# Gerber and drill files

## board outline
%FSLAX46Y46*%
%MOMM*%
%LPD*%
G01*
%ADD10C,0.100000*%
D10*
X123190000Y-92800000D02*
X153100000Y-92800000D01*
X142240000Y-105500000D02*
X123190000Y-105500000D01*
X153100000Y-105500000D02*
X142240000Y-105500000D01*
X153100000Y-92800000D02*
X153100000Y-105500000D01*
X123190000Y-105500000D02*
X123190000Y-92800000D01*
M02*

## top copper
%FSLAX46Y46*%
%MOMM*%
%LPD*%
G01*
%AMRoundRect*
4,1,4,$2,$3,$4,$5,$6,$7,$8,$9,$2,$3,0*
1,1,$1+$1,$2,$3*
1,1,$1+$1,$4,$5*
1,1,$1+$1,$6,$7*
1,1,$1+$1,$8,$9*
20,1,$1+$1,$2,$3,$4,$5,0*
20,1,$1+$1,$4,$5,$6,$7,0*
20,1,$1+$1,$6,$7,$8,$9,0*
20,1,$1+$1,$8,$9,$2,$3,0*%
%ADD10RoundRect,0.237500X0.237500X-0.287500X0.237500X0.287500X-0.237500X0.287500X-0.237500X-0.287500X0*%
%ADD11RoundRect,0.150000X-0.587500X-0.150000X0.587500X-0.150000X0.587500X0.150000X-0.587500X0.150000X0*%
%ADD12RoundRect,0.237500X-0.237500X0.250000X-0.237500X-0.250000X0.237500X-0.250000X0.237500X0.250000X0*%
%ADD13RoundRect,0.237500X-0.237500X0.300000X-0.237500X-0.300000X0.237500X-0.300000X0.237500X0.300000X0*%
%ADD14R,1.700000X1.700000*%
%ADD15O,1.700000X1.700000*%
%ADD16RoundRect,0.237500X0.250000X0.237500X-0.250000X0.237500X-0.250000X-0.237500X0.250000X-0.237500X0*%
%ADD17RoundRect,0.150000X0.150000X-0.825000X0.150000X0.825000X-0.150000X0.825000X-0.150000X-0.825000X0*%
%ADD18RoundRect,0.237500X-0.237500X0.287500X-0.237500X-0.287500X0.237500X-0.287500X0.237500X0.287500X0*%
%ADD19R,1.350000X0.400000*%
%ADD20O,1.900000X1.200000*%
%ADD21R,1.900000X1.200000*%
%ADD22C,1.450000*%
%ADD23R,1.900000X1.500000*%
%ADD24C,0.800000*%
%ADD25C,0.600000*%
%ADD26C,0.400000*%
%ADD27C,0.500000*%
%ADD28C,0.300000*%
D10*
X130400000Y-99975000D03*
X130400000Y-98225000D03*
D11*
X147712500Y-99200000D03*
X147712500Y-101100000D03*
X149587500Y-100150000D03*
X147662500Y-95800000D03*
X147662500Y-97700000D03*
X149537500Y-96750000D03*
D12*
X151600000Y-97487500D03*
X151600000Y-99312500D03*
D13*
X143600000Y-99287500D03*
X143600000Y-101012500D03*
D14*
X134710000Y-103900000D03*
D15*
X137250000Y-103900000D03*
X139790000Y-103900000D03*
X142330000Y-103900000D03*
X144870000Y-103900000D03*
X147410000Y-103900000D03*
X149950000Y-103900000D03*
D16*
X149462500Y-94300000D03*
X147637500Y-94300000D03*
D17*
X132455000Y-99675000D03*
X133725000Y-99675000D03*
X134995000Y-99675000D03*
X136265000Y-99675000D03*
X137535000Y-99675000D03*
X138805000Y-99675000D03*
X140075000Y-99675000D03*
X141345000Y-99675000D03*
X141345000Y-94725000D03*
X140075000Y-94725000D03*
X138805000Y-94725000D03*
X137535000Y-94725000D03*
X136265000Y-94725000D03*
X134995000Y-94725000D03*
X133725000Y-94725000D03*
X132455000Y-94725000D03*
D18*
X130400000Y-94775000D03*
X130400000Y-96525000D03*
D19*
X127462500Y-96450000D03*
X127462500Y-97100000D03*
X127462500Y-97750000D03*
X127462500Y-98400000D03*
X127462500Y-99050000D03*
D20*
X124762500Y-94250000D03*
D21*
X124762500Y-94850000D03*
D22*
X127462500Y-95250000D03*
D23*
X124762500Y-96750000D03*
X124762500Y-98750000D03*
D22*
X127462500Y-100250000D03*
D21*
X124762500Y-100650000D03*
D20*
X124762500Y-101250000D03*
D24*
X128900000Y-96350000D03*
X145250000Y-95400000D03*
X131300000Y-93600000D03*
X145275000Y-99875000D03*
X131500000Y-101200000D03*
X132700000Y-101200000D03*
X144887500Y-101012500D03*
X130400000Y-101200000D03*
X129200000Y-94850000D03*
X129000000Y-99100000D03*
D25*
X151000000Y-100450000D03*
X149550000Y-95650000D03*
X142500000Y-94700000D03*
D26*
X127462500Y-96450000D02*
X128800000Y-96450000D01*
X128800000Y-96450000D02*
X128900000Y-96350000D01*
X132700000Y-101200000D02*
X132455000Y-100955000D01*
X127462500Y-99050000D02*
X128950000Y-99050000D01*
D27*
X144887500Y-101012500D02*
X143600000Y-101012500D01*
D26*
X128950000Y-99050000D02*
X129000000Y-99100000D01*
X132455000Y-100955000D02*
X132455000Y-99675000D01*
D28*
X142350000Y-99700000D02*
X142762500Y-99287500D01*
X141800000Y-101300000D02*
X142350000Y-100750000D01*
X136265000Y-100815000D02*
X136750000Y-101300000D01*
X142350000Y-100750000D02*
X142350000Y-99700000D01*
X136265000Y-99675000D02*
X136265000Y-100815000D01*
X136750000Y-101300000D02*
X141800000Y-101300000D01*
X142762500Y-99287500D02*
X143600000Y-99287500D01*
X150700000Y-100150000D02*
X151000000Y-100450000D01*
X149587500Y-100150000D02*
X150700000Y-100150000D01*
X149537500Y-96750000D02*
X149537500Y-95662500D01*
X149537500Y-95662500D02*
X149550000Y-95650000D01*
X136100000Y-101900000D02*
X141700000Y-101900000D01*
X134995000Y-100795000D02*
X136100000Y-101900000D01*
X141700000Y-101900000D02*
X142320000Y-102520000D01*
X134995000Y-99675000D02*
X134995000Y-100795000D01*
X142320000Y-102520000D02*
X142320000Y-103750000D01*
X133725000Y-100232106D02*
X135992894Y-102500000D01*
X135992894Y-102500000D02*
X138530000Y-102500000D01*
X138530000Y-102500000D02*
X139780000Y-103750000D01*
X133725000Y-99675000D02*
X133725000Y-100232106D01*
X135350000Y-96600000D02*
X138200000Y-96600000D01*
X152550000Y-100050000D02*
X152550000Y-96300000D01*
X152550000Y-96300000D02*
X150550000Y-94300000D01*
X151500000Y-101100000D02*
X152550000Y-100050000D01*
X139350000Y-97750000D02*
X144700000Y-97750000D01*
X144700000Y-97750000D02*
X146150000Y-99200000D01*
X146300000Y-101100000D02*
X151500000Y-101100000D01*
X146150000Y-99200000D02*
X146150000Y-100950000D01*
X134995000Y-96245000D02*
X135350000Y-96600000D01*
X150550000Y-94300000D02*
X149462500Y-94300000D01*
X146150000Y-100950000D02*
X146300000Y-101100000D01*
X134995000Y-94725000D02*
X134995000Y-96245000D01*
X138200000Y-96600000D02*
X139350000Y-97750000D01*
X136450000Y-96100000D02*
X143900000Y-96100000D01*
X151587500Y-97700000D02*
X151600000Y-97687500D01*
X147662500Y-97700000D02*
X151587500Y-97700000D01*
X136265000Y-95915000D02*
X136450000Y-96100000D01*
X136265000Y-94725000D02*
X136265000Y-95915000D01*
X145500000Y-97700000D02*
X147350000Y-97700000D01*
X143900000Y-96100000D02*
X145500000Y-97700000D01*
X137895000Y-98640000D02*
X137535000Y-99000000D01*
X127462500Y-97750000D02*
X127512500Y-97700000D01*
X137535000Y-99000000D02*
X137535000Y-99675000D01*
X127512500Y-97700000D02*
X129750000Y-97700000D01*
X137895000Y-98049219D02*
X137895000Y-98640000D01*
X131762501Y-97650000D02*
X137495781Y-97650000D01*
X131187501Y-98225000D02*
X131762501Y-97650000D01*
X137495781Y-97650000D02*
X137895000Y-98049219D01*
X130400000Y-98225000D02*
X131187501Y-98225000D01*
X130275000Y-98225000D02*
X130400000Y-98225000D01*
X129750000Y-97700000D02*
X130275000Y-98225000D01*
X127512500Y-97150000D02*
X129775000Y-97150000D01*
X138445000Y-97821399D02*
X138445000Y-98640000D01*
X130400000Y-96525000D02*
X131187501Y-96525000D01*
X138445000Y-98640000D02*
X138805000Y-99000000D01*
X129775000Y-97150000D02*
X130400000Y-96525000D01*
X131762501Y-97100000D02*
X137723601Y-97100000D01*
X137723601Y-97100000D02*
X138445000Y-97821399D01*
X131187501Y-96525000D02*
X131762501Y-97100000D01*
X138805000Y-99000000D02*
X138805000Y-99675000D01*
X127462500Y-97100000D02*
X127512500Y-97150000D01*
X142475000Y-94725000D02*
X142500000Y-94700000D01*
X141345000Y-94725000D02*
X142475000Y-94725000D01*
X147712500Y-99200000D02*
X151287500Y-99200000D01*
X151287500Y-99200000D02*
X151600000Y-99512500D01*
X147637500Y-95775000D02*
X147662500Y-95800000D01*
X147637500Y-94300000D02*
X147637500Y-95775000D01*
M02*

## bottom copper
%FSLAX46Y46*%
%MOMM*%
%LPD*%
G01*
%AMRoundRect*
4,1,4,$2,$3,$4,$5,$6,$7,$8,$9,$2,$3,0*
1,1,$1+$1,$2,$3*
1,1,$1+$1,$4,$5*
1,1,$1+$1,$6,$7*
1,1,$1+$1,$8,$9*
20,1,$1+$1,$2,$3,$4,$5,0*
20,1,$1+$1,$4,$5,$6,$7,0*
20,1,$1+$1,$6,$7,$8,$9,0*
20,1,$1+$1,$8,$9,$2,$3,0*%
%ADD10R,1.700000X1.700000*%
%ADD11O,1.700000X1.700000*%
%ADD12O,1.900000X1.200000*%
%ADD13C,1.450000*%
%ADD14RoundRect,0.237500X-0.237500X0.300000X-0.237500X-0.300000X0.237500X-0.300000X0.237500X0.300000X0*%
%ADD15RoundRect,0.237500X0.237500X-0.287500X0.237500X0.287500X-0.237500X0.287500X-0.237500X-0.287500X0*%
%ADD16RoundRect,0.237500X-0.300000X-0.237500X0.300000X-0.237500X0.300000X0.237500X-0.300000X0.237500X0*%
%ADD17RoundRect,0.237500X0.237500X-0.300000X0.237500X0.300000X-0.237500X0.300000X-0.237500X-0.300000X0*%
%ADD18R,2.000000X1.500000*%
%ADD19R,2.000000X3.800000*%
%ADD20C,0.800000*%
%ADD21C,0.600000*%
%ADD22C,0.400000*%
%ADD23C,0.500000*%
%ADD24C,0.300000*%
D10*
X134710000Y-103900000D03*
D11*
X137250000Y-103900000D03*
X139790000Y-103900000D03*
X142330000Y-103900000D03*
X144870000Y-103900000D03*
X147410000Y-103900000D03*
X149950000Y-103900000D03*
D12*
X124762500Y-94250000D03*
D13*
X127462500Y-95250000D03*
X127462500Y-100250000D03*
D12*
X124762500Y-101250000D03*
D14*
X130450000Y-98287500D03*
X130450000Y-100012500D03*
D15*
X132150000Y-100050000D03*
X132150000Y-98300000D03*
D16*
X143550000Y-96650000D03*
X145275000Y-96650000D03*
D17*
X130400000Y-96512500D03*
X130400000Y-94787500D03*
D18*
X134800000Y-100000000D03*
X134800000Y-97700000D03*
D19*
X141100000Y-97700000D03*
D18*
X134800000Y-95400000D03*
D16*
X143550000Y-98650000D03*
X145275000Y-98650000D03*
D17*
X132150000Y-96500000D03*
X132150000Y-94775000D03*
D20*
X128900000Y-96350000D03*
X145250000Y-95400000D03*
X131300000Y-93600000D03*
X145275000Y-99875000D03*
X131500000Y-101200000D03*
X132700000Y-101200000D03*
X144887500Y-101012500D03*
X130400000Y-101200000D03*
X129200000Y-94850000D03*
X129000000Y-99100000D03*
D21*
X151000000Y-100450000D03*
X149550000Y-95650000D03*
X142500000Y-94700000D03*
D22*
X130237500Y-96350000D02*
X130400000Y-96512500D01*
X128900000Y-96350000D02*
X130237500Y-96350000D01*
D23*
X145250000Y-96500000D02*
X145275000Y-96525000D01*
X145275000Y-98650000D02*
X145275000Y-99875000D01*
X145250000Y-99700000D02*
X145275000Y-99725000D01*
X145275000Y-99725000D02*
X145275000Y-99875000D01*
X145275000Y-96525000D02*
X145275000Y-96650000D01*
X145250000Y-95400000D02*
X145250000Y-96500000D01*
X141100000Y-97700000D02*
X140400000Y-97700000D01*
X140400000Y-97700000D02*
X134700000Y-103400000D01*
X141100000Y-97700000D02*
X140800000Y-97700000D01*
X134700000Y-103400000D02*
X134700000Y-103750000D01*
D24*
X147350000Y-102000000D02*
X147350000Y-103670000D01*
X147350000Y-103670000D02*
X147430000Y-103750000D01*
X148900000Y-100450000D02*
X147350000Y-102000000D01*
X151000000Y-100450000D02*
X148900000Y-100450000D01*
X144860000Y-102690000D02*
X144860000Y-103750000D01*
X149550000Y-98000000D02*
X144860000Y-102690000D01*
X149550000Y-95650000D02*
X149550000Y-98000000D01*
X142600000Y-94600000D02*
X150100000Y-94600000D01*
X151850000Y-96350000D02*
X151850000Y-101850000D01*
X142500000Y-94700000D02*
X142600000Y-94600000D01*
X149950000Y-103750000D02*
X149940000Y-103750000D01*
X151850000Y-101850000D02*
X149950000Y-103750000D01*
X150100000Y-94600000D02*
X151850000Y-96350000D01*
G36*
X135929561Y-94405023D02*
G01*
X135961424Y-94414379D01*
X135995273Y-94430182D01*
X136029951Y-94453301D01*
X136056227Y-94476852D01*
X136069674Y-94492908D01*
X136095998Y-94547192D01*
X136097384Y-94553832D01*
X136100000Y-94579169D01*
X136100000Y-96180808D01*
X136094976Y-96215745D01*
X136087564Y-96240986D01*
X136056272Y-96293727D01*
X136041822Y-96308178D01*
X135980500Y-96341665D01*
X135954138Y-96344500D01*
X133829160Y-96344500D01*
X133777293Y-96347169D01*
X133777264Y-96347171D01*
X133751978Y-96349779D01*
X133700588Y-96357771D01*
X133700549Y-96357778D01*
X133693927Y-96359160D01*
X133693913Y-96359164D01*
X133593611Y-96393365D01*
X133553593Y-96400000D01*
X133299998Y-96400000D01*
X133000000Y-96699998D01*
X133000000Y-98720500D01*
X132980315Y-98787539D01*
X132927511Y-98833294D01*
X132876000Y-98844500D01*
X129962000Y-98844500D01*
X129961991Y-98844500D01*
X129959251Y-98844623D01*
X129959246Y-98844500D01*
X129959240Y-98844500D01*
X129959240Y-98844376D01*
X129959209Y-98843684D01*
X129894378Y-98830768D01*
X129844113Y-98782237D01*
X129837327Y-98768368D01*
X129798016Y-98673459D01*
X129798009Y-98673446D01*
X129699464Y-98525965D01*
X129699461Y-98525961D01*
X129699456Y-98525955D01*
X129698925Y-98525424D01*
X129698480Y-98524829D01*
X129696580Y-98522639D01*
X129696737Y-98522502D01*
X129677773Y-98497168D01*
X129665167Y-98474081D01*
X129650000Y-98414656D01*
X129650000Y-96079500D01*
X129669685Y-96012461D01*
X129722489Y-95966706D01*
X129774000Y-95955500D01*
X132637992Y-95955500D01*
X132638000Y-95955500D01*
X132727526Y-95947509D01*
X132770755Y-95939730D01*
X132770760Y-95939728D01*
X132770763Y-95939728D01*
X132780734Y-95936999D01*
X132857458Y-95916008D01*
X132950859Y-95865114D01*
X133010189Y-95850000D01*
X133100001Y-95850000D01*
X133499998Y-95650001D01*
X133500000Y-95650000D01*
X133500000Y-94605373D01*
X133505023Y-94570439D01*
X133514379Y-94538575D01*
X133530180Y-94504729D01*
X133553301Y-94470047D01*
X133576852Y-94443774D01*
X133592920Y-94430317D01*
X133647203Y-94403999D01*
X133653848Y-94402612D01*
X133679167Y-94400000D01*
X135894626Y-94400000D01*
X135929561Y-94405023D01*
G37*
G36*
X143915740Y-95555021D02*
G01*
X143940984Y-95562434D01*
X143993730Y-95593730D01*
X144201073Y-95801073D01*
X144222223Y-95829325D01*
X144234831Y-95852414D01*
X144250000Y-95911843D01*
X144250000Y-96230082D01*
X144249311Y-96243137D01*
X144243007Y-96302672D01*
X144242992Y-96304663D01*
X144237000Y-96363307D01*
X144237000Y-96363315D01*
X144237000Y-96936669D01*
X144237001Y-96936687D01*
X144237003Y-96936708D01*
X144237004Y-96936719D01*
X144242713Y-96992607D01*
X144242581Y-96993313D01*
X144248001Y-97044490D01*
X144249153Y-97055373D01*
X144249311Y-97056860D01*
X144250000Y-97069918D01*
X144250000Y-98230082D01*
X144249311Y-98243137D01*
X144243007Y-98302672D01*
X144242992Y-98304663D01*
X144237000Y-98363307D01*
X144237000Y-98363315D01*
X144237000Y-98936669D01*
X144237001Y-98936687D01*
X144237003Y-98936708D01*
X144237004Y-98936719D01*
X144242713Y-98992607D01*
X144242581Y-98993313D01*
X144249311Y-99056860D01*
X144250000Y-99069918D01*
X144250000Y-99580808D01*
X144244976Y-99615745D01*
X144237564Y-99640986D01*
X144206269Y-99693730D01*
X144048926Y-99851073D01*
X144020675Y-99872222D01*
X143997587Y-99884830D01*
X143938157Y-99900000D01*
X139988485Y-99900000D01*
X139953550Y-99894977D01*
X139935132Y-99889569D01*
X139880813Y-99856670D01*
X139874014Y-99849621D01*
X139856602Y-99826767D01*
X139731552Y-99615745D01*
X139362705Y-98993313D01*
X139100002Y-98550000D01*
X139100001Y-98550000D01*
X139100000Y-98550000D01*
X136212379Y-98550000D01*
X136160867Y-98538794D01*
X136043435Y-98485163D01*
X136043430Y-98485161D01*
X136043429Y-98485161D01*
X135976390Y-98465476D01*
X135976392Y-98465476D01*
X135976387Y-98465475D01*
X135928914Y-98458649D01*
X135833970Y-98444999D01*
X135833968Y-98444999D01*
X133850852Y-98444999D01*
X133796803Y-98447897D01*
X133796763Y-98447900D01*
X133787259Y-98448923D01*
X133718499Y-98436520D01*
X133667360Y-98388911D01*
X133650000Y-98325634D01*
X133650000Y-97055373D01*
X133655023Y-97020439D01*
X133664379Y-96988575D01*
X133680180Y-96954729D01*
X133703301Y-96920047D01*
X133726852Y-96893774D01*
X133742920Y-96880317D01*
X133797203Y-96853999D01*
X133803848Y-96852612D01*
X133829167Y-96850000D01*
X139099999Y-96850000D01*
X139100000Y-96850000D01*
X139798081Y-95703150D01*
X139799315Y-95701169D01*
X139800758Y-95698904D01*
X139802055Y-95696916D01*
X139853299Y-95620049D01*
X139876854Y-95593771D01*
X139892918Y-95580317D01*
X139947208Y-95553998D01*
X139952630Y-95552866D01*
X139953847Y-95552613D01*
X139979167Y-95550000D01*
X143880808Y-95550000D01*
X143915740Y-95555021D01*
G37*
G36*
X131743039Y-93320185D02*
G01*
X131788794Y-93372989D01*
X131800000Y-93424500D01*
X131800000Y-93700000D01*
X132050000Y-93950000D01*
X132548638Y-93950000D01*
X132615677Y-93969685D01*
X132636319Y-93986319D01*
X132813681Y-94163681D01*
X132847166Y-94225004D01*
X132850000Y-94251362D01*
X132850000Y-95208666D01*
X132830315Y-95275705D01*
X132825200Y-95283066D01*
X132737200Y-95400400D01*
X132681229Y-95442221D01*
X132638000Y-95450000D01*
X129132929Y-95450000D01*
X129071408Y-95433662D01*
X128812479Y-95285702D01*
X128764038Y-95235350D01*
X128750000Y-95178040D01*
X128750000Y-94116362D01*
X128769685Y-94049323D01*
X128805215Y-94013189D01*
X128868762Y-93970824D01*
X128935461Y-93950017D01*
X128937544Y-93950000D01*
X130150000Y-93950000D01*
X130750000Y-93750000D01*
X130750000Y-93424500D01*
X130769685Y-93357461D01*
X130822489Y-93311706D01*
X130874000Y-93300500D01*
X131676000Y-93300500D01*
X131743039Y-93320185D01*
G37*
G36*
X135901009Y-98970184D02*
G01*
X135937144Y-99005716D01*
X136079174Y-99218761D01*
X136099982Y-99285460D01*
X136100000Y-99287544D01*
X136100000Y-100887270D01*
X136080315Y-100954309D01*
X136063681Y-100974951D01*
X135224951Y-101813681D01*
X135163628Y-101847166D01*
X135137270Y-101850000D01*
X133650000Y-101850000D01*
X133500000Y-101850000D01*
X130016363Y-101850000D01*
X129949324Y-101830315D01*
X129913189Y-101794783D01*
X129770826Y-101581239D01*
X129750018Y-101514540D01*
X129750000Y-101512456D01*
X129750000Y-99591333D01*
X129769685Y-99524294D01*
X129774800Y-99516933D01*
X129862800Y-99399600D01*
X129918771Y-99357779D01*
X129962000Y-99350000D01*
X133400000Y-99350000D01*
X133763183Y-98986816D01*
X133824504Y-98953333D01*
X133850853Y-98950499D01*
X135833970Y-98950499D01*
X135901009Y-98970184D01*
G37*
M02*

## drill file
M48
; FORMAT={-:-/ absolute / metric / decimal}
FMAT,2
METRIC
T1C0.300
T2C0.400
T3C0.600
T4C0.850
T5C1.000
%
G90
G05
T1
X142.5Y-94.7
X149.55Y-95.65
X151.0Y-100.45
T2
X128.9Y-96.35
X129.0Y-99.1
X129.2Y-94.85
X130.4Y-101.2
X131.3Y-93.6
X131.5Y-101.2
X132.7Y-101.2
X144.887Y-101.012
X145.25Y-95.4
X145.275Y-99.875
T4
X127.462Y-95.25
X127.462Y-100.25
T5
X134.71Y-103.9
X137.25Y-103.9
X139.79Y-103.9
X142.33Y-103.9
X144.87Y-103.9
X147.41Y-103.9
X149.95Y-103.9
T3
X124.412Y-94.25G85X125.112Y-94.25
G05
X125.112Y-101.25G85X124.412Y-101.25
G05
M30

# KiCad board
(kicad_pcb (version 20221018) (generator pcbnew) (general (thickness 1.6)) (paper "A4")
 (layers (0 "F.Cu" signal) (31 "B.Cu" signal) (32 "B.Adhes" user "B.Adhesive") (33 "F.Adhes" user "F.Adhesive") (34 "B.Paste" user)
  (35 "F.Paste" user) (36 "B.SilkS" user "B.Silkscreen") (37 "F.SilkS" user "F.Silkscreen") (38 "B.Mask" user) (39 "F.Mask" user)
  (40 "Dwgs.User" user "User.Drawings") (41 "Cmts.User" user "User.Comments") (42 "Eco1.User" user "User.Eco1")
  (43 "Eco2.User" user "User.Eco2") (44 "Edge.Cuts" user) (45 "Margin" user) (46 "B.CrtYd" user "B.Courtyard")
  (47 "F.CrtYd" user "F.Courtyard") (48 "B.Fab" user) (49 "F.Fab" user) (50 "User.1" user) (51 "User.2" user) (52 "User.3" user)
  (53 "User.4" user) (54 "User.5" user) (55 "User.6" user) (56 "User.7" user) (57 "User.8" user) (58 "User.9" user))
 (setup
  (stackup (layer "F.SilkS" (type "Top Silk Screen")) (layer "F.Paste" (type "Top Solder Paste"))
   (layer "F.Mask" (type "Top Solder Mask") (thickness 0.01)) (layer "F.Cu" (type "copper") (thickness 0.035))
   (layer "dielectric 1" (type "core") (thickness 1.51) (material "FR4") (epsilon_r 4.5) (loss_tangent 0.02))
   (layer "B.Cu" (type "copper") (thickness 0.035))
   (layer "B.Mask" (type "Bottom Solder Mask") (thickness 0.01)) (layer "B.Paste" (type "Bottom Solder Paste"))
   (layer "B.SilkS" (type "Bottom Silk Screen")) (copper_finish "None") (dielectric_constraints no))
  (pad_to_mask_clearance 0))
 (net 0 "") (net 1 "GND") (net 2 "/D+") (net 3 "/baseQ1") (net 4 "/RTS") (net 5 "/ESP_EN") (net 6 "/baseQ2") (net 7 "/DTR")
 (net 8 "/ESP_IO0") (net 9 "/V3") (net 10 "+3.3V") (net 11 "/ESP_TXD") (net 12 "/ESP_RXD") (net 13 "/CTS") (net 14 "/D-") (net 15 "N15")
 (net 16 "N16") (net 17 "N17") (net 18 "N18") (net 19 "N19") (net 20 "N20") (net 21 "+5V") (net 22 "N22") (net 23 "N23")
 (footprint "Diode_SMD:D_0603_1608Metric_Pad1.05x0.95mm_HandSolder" (layer "F.Cu") (at 130.4 99.1 90)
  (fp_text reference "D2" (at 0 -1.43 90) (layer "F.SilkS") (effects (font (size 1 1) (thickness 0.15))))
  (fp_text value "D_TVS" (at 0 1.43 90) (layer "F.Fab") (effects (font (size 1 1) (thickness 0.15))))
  (pad "1" smd roundrect (at -0.875 0 90) (size 1.05 0.95) (layers "F.Cu" "F.Paste" "F.Mask") (roundrect_rratio 0.25) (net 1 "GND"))
  (pad "2" smd roundrect (at 0.875 0 90) (size 1.05 0.95) (layers "F.Cu" "F.Paste" "F.Mask") (roundrect_rratio 0.25) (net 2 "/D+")))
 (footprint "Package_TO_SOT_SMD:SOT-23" (layer "F.Cu") (at 148.65 100.15)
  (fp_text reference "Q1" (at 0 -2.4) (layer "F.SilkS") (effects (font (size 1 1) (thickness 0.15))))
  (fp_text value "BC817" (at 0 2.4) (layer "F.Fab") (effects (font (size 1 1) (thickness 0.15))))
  (pad "1" smd roundrect (at -0.9375 -0.95) (size 1.475 0.6) (layers "F.Cu" "F.Paste" "F.Mask") (roundrect_rratio 0.25) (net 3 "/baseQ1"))
  (pad "2" smd roundrect (at -0.9375 0.95) (size 1.475 0.6) (layers "F.Cu" "F.Paste" "F.Mask") (roundrect_rratio 0.25) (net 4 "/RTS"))
  (pad "3" smd roundrect (at 0.9375 0) (size 1.475 0.6) (layers "F.Cu" "F.Paste" "F.Mask") (roundrect_rratio 0.25) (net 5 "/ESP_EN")))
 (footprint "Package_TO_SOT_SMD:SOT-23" (layer "F.Cu") (at 148.6 96.75)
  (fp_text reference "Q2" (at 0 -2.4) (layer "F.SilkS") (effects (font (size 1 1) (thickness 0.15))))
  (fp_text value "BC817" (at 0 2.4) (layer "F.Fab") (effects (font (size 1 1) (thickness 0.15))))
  (pad "1" smd roundrect (at -0.9375 -0.95) (size 1.475 0.6) (layers "F.Cu" "F.Paste" "F.Mask") (roundrect_rratio 0.25) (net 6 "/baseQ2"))
  (pad "2" smd roundrect (at -0.9375 0.95) (size 1.475 0.6) (layers "F.Cu" "F.Paste" "F.Mask") (roundrect_rratio 0.25) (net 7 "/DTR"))
  (pad "3" smd roundrect (at 0.9375 0) (size 1.475 0.6) (layers "F.Cu" "F.Paste" "F.Mask") (roundrect_rratio 0.25) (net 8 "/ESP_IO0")))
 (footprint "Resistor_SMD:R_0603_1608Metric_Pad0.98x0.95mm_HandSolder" (layer "F.Cu") (at 151.6 98.4 -90)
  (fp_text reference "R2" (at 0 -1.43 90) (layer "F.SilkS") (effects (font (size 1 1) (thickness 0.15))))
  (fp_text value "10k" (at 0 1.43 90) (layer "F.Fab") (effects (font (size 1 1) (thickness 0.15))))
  (pad "1" smd roundrect (at -0.9125 0 270) (size 0.975 0.95) (layers "F.Cu" "F.Paste" "F.Mask") (roundrect_rratio 0.25) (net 7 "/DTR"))
  (pad "2" smd roundrect (at 0.9125 0 270) (size 0.975 0.95) (layers "F.Cu" "F.Paste" "F.Mask") (roundrect_rratio 0.25) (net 3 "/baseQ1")))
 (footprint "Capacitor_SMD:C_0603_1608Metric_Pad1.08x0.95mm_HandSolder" (layer "F.Cu") (at 143.6 100.15 -90)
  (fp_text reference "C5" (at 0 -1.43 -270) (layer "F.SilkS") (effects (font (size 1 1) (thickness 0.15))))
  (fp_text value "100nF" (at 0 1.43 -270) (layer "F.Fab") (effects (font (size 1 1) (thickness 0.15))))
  (pad "1" smd roundrect (at -0.8625 0 270) (size 1.075 0.95) (layers "F.Cu" "F.Paste" "F.Mask") (roundrect_rratio 0.25) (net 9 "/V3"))
  (pad "2" smd roundrect (at 0.8625 0 270) (size 1.075 0.95) (layers "F.Cu" "F.Paste" "F.Mask") (roundrect_rratio 0.25) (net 1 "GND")))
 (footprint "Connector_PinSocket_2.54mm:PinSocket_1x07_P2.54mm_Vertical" (layer "F.Cu") (at 134.71 103.9 90)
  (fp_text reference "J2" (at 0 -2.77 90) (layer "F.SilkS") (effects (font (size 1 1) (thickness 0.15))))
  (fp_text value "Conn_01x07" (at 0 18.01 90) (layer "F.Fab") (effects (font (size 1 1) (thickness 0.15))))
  (pad "1" thru_hole rect (at 0 0 90) (size 1.7 1.7) (drill 1) (layers "*.Cu" "*.Mask") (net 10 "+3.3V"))
  (pad "2" thru_hole oval (at 0 2.54 90) (size 1.7 1.7) (drill 1) (layers "*.Cu" "*.Mask") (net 1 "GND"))
  (pad "3" thru_hole oval (at 0 5.08 90) (size 1.7 1.7) (drill 1) (layers "*.Cu" "*.Mask") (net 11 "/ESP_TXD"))
  (pad "4" thru_hole oval (at 0 7.62 90) (size 1.7 1.7) (drill 1) (layers "*.Cu" "*.Mask") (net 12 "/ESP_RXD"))
  (pad "5" thru_hole oval (at 0 10.16 90) (size 1.7 1.7) (drill 1) (layers "*.Cu" "*.Mask") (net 8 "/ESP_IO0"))
  (pad "6" thru_hole oval (at 0 12.7 90) (size 1.7 1.7) (drill 1) (layers "*.Cu" "*.Mask") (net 5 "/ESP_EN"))
  (pad "7" thru_hole oval (at 0 15.24 90) (size 1.7 1.7) (drill 1) (layers "*.Cu" "*.Mask") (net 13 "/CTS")))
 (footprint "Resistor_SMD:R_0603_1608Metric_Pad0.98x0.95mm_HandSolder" (layer "F.Cu") (at 148.55 94.3 180)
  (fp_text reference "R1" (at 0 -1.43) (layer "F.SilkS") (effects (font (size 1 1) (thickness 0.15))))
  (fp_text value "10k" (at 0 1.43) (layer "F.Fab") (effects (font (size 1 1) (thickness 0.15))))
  (pad "1" smd roundrect (at -0.9125 0 180) (size 0.975 0.95) (layers "F.Cu" "F.Paste" "F.Mask") (roundrect_rratio 0.25) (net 4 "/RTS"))
  (pad "2" smd roundrect (at 0.9125 0 180) (size 0.975 0.95) (layers "F.Cu" "F.Paste" "F.Mask") (roundrect_rratio 0.25) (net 6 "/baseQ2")))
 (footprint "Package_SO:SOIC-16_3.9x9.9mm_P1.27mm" (layer "F.Cu") (at 136.9 97.2 90)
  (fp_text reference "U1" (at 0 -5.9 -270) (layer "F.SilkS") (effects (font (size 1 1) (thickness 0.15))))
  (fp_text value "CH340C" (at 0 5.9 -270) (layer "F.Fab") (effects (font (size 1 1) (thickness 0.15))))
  (pad "1" smd roundrect (at -2.475 -4.445 90) (size 1.95 0.6) (layers "F.Cu" "F.Paste" "F.Mask") (roundrect_rratio 0.25) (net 1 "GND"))
  (pad "2" smd roundrect (at -2.475 -3.175 90) (size 1.95 0.6) (layers "F.Cu" "F.Paste" "F.Mask") (roundrect_rratio 0.25)
   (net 11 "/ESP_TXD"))
  (pad "3" smd roundrect (at -2.475 -1.905 90) (size 1.95 0.6) (layers "F.Cu" "F.Paste" "F.Mask") (roundrect_rratio 0.25)
   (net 12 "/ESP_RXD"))
  (pad "4" smd roundrect (at -2.475 -0.635 90) (size 1.95 0.6) (layers "F.Cu" "F.Paste" "F.Mask") (roundrect_rratio 0.25) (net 9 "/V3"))
  (pad "5" smd roundrect (at -2.475 0.635 90) (size 1.95 0.6) (layers "F.Cu" "F.Paste" "F.Mask") (roundrect_rratio 0.25) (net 2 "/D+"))
  (pad "6" smd roundrect (at -2.475 1.905 90) (size 1.95 0.6) (layers "F.Cu" "F.Paste" "F.Mask") (roundrect_rratio 0.25) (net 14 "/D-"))
  (pad "7" smd roundrect (at -2.475 3.175 90) (size 1.95 0.6) (layers "F.Cu" "F.Paste" "F.Mask") (roundrect_rratio 0.25) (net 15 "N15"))
  (pad "8" smd roundrect (at -2.475 4.445 90) (size 1.95 0.6) (layers "F.Cu" "F.Paste" "F.Mask") (roundrect_rratio 0.25) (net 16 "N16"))
  (pad "9" smd roundrect (at 2.475 4.445 90) (size 1.95 0.6) (layers "F.Cu" "F.Paste" "F.Mask") (roundrect_rratio 0.25) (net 13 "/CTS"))
  (pad "10" smd roundrect (at 2.475 3.175 90) (size 1.95 0.6) (layers "F.Cu" "F.Paste" "F.Mask") (roundrect_rratio 0.25) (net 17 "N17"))
  (pad "11" smd roundrect (at 2.475 1.905 90) (size 1.95 0.6) (layers "F.Cu" "F.Paste" "F.Mask") (roundrect_rratio 0.25) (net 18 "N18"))
  (pad "12" smd roundrect (at 2.475 0.635 90) (size 1.95 0.6) (layers "F.Cu" "F.Paste" "F.Mask") (roundrect_rratio 0.25) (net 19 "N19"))
  (pad "13" smd roundrect (at 2.475 -0.635 90) (size 1.95 0.6) (layers "F.Cu" "F.Paste" "F.Mask") (roundrect_rratio 0.25) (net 7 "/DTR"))
  (pad "14" smd roundrect (at 2.475 -1.905 90) (size 1.95 0.6) (layers "F.Cu" "F.Paste" "F.Mask") (roundrect_rratio 0.25) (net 4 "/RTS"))
  (pad "15" smd roundrect (at 2.475 -3.175 90) (size 1.95 0.6) (layers "F.Cu" "F.Paste" "F.Mask") (roundrect_rratio 0.25) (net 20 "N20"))
  (pad "16" smd roundrect (at 2.475 -4.445 90) (size 1.95 0.6) (layers "F.Cu" "F.Paste" "F.Mask") (roundrect_rratio 0.25) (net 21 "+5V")))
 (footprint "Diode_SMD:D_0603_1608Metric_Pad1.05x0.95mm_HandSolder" (layer "F.Cu") (at 130.4 95.65 -90)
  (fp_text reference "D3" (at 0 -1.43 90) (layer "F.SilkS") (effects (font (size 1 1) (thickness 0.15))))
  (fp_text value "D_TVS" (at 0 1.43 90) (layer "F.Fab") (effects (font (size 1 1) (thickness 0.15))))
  (pad "1" smd roundrect (at -0.875 0 270) (size 1.05 0.95) (layers "F.Cu" "F.Paste" "F.Mask") (roundrect_rratio 0.25) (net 1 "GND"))
  (pad "2" smd roundrect (at 0.875 0 270) (size 1.05 0.95) (layers "F.Cu" "F.Paste" "F.Mask") (roundrect_rratio 0.25) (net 14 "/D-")))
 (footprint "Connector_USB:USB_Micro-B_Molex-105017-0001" (layer "F.Cu") (at 126 97.75 -90)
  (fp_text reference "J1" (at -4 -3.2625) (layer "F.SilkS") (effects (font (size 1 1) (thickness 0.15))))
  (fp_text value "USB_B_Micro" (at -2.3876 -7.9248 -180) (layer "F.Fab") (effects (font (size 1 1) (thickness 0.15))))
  (pad "1" smd rect (at -1.3 -1.4625 270) (size 0.4 1.35) (layers "F.Cu" "F.Paste" "F.Mask") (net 21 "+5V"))
  (pad "2" smd rect (at -0.65 -1.4625 270) (size 0.4 1.35) (layers "F.Cu" "F.Paste" "F.Mask") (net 14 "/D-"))
  (pad "3" smd rect (at 0 -1.4625 270) (size 0.4 1.35) (layers "F.Cu" "F.Paste" "F.Mask") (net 2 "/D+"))
  (pad "4" smd rect (at 0.65 -1.4625 270) (size 0.4 1.35) (layers "F.Cu" "F.Paste" "F.Mask") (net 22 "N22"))
  (pad "5" smd rect (at 1.3 -1.4625 270) (size 0.4 1.35) (layers "F.Cu" "F.Paste" "F.Mask") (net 1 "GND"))
  (pad "6" thru_hole oval (at -3.5 1.2375 90) (size 1.2 1.9) (drill oval 0.6 1.3) (layers "*.Cu" "*.Mask") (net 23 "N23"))
  (pad "6" smd rect (at -2.9 1.2375 270) (size 1.2 1.9) (layers "F.Cu" "F.Mask") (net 23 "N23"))
  (pad "6" thru_hole circle (at -2.5 -1.4625 270) (size 1.45 1.45) (drill 0.85) (layers "*.Cu" "*.Mask") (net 23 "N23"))
  (pad "6" smd rect (at -1 1.2375 270) (size 1.5 1.9) (layers "F.Cu" "F.Paste" "F.Mask") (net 23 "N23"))
  (pad "6" smd rect (at 1 1.2375 270) (size 1.5 1.9) (layers "F.Cu" "F.Paste" "F.Mask") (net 23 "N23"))
  (pad "6" thru_hole circle (at 2.5 -1.4625 270) (size 1.45 1.45) (drill 0.85) (layers "*.Cu" "*.Mask") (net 23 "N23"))
  (pad "6" smd rect (at 2.9 1.2375 270) (size 1.2 1.9) (layers "F.Cu" "F.Mask") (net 23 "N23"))
  (pad "6" thru_hole oval (at 3.5 1.2375 270) (size 1.2 1.9) (drill oval 0.6 1.3) (layers "*.Cu" "*.Mask") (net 23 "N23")))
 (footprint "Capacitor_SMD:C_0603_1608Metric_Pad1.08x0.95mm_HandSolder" (layer "B.Cu") (at 130.45 99.15 -90)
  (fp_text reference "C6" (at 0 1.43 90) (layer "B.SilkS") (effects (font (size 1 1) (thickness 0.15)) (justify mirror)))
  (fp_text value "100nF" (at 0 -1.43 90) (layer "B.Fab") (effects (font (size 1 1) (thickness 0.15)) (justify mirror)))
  (pad "1" smd roundrect (at -0.8625 0 270) (size 1.075 0.95) (layers "B.Cu" "B.Paste" "B.Mask") (roundrect_rratio 0.25) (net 21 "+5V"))
  (pad "2" smd roundrect (at 0.8625 0 270) (size 1.075 0.95) (layers "B.Cu" "B.Paste" "B.Mask") (roundrect_rratio 0.25) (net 1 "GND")))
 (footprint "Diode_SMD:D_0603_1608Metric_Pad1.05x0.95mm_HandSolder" (layer "B.Cu") (at 132.15 99.175 90)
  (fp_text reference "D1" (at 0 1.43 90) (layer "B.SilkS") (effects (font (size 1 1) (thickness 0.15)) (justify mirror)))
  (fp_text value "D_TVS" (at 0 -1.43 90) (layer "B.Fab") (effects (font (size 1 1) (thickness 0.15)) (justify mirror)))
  (pad "1" smd roundrect (at -0.875 0 90) (size 1.05 0.95) (layers "B.Cu" "B.Paste" "B.Mask") (roundrect_rratio 0.25) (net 1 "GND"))
  (pad "2" smd roundrect (at 0.875 0 90) (size 1.05 0.95) (layers "B.Cu" "B.Paste" "B.Mask") (roundrect_rratio 0.25) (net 21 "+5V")))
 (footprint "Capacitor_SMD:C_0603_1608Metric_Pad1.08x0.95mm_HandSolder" (layer "B.Cu") (at 144.4125 96.65)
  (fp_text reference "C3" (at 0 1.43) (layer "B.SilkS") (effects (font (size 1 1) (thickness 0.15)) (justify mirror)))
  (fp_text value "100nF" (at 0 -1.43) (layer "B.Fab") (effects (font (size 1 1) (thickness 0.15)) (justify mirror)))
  (pad "1" smd roundrect (at -0.8625 0) (size 1.075 0.95) (layers "B.Cu" "B.Paste" "B.Mask") (roundrect_rratio 0.25) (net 10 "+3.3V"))
  (pad "2" smd roundrect (at 0.8625 0) (size 1.075 0.95) (layers "B.Cu" "B.Paste" "B.Mask") (roundrect_rratio 0.25) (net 1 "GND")))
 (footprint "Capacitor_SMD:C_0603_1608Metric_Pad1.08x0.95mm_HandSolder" (layer "B.Cu") (at 130.4 95.65 90)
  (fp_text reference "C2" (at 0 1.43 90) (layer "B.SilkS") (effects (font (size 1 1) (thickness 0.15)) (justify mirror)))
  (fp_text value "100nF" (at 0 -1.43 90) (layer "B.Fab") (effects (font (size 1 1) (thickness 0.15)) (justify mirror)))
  (pad "1" smd roundrect (at -0.8625 0 90) (size 1.075 0.95) (layers "B.Cu" "B.Paste" "B.Mask") (roundrect_rratio 0.25) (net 21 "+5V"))
  (pad "2" smd roundrect (at 0.8625 0 90) (size 1.075 0.95) (layers "B.Cu" "B.Paste" "B.Mask") (roundrect_rratio 0.25) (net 1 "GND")))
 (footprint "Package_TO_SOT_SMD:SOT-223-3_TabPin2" (layer "B.Cu") (at 137.95 97.7)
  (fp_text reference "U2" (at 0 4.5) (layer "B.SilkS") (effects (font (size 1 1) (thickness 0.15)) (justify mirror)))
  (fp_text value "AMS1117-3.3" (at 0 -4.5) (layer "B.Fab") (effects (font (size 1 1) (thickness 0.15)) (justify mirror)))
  (pad "1" smd rect (at -3.15 2.3) (size 2 1.5) (layers "B.Cu" "B.Paste" "B.Mask") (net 1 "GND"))
  (pad "2" smd rect (at -3.15 0) (size 2 1.5) (layers "B.Cu" "B.Paste" "B.Mask") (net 10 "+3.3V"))
  (pad "2" smd rect (at 3.15 0) (size 2 3.8) (layers "B.Cu" "B.Paste" "B.Mask") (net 10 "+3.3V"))
  (pad "3" smd rect (at -3.15 -2.3) (size 2 1.5) (layers "B.Cu" "B.Paste" "B.Mask") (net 21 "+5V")))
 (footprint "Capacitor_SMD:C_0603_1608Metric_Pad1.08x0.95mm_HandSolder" (layer "B.Cu") (at 144.4125 98.65)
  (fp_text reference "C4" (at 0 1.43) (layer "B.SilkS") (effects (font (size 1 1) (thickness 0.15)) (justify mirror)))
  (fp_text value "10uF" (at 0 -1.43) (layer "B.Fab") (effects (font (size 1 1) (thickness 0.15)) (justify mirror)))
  (pad "1" smd roundrect (at -0.8625 0) (size 1.075 0.95) (layers "B.Cu" "B.Paste" "B.Mask") (roundrect_rratio 0.25) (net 10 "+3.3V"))
  (pad "2" smd roundrect (at 0.8625 0) (size 1.075 0.95) (layers "B.Cu" "B.Paste" "B.Mask") (roundrect_rratio 0.25) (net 1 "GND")))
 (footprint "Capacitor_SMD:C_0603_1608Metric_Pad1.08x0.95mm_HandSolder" (layer "B.Cu") (at 132.15 95.6375 90)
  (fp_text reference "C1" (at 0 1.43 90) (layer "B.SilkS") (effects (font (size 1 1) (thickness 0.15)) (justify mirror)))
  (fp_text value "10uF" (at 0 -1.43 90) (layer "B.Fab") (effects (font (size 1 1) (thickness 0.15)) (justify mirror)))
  (pad "1" smd roundrect (at -0.8625 0 90) (size 1.075 0.95) (layers "B.Cu" "B.Paste" "B.Mask") (roundrect_rratio 0.25) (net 21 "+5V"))
  (pad "2" smd roundrect (at 0.8625 0 90) (size 1.075 0.95) (layers "B.Cu" "B.Paste" "B.Mask") (roundrect_rratio 0.25) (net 1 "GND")))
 (gr_line (start 123.19 92.8) (end 153.1 92.8) (stroke (width 0.1) (type default)) (layer "Edge.Cuts"))
 (gr_line (start 142.24 105.5) (end 123.19 105.5) (stroke (width 0.1) (type default)) (layer "Edge.Cuts"))
 (gr_line (start 153.1 105.5) (end 142.24 105.5) (stroke (width 0.1) (type default)) (layer "Edge.Cuts"))
 (gr_line (start 153.1 92.8) (end 153.1 105.5) (stroke (width 0.1) (type default)) (layer "Edge.Cuts"))
 (gr_line (start 123.19 105.5) (end 123.19 92.8) (stroke (width 0.1) (type default)) (layer "Edge.Cuts"))
 (segment (start 127.4625 96.45) (end 128.8 96.45) (width 0.4) (layer "F.Cu") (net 21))
 (segment (start 128.8 96.45) (end 128.9 96.35) (width 0.4) (layer "F.Cu") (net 21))
 (via (at 128.9 96.35) (size 0.8) (drill 0.4) (layers "F.Cu" "B.Cu") (free) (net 21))
 (segment (start 130.2375 96.35) (end 130.4 96.5125) (width 0.4) (layer "B.Cu") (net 21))
 (segment (start 128.9 96.35) (end 130.2375 96.35) (width 0.4) (layer "B.Cu") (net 21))
 (segment (start 132.7 101.2) (end 132.455 100.955) (width 0.4) (layer "F.Cu") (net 1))
 (segment (start 127.4625 99.05) (end 128.95 99.05) (width 0.4) (layer "F.Cu") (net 1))
 (segment (start 144.8875 101.0125) (end 143.6 101.0125) (width 0.5) (layer "F.Cu") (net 1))
 (segment (start 128.95 99.05) (end 129 99.1) (width 0.4) (layer "F.Cu") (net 1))
 (segment (start 132.455 100.955) (end 132.455 99.675) (width 0.4) (layer "F.Cu") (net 1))
 (via (at 145.25 95.4) (size 0.8) (drill 0.4) (layers "F.Cu" "B.Cu") (free) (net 1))
 (via (at 131.3 93.6) (size 0.8) (drill 0.4) (layers "F.Cu" "B.Cu") (free) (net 1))
 (via (at 145.275 99.875) (size 0.8) (drill 0.4) (layers "F.Cu" "B.Cu") (free) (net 1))
 (via (at 131.5 101.2) (size 0.8) (drill 0.4) (layers "F.Cu" "B.Cu") (free) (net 1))
 (via (at 132.7 101.2) (size 0.8) (drill 0.4) (layers "F.Cu" "B.Cu") (free) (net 1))
 (via (at 144.8875 101.0125) (size 0.8) (drill 0.4) (layers "F.Cu" "B.Cu") (free) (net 1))
 (via (at 130.4 101.2) (size 0.8) (drill 0.4) (layers "F.Cu" "B.Cu") (free) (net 1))
 (via (at 129.2 94.85) (size 0.8) (drill 0.4) (layers "F.Cu" "B.Cu") (free) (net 1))
 (via (at 129 99.1) (size 0.8) (drill 0.4) (layers "F.Cu" "B.Cu") (free) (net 1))
 (segment (start 145.25 96.5) (end 145.275 96.525) (width 0.5) (layer "B.Cu") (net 1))
 (segment (start 145.275 98.65) (end 145.275 99.875) (width 0.5) (layer "B.Cu") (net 1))
 (segment (start 145.25 99.7) (end 145.275 99.725) (width 0.5) (layer "B.Cu") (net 1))
 (segment (start 145.275 99.725) (end 145.275 99.875) (width 0.5) (layer "B.Cu") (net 1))
 (segment (start 145.275 96.525) (end 145.275 96.65) (width 0.5) (layer "B.Cu") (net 1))
 (segment (start 145.25 95.4) (end 145.25 96.5) (width 0.5) (layer "B.Cu") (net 1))
 (segment (start 141.1 97.7) (end 140.4 97.7) (width 0.5) (layer "B.Cu") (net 10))
 (segment (start 140.4 97.7) (end 134.7 103.4) (width 0.5) (layer "B.Cu") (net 10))
 (segment (start 141.1 97.7) (end 140.8 97.7) (width 0.5) (layer "B.Cu") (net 10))
 (segment (start 134.7 103.4) (end 134.7 103.75) (width 0.5) (layer "B.Cu") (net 10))
 (segment (start 142.35 99.7) (end 142.7625 99.2875) (width 0.3) (layer "F.Cu") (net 9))
 (segment (start 141.8 101.3) (end 142.35 100.75) (width 0.3) (layer "F.Cu") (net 9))
 (segment (start 136.265 100.815) (end 136.75 101.3) (width 0.3) (layer "F.Cu") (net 9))
 (segment (start 142.35 100.75) (end 142.35 99.7) (width 0.3) (layer "F.Cu") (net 9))
 (segment (start 136.265 99.675) (end 136.265 100.815) (width 0.3) (layer "F.Cu") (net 9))
 (segment (start 136.75 101.3) (end 141.8 101.3) (width 0.3) (layer "F.Cu") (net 9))
 (segment (start 142.7625 99.2875) (end 143.6 99.2875) (width 0.3) (layer "F.Cu") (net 9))
 (segment (start 150.7 100.15) (end 151 100.45) (width 0.3) (layer "F.Cu") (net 5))
 (segment (start 149.5875 100.15) (end 150.7 100.15) (width 0.3) (layer "F.Cu") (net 5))
 (via (at 151 100.45) (size 0.6) (drill 0.3) (layers "F.Cu" "B.Cu") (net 5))
 (segment (start 147.35 102) (end 147.35 103.67) (width 0.3) (layer "B.Cu") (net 5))
 (segment (start 147.35 103.67) (end 147.43 103.75) (width 0.3) (layer "B.Cu") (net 5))
 (segment (start 148.9 100.45) (end 147.35 102) (width 0.3) (layer "B.Cu") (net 5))
 (segment (start 151 100.45) (end 148.9 100.45) (width 0.3) (layer "B.Cu") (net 5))
 (segment (start 149.5375 96.75) (end 149.5375 95.6625) (width 0.3) (layer "F.Cu") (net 8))
 (segment (start 149.5375 95.6625) (end 149.55 95.65) (width 0.3) (layer "F.Cu") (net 8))
 (via (at 149.55 95.65) (size 0.6) (drill 0.3) (layers "F.Cu" "B.Cu") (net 8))
 (segment (start 144.86 102.69) (end 144.86 103.75) (width 0.3) (layer "B.Cu") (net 8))
 (segment (start 149.55 98) (end 144.86 102.69) (width 0.3) (layer "B.Cu") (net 8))
 (segment (start 149.55 95.65) (end 149.55 98) (width 0.3) (layer "B.Cu") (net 8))
 (segment (start 136.1 101.9) (end 141.7 101.9) (width 0.3) (layer "F.Cu") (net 12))
 (segment (start 134.995 100.795) (end 136.1 101.9) (width 0.3) (layer "F.Cu") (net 12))
 (segment (start 141.7 101.9) (end 142.32 102.52) (width 0.3) (layer "F.Cu") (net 12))
 (segment (start 134.995 99.675) (end 134.995 100.795) (width 0.3) (layer "F.Cu") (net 12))
 (segment (start 142.32 102.52) (end 142.32 103.75) (width 0.3) (layer "F.Cu") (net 12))
 (segment (start 133.725 100.232106) (end 135.992894 102.5) (width 0.3) (layer "F.Cu") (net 11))
 (segment (start 135.992894 102.5) (end 138.53 102.5) (width 0.3) (layer "F.Cu") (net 11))
 (segment (start 138.53 102.5) (end 139.78 103.75) (width 0.3) (layer "F.Cu") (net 11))
 (segment (start 133.725 99.675) (end 133.725 100.232106) (width 0.3) (layer "F.Cu") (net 11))
 (segment (start 135.35 96.6) (end 138.2 96.6) (width 0.3) (layer "F.Cu") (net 4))
 (segment (start 152.55 100.05) (end 152.55 96.3) (width 0.3) (layer "F.Cu") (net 4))
 (segment (start 152.55 96.3) (end 150.55 94.3) (width 0.3) (layer "F.Cu") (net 4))
 (segment (start 151.5 101.1) (end 152.55 100.05) (width 0.3) (layer "F.Cu") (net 4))
 (segment (start 139.35 97.75) (end 144.7 97.75) (width 0.3) (layer "F.Cu") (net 4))
 (segment (start 144.7 97.75) (end 146.15 99.2) (width 0.3) (layer "F.Cu") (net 4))
 (segment (start 146.3 101.1) (end 151.5 101.1) (width 0.3) (layer "F.Cu") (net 4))
 (segment (start 146.15 99.2) (end 146.15 100.95) (width 0.3) (layer "F.Cu") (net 4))
 (segment (start 134.995 96.245) (end 135.35 96.6) (width 0.3) (layer "F.Cu") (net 4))
 (segment (start 150.55 94.3) (end 149.4625 94.3) (width 0.3) (layer "F.Cu") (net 4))
 (segment (start 146.15 100.95) (end 146.3 101.1) (width 0.3) (layer "F.Cu") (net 4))
 (segment (start 134.995 94.725) (end 134.995 96.245) (width 0.3) (layer "F.Cu") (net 4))
 (segment (start 138.2 96.6) (end 139.35 97.75) (width 0.3) (layer "F.Cu") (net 4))
 (segment (start 136.45 96.1) (end 143.9 96.1) (width 0.3) (layer "F.Cu") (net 7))
 (segment (start 151.5875 97.7) (end 151.6 97.6875) (width 0.3) (layer "F.Cu") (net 7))
 (segment (start 147.6625 97.7) (end 151.5875 97.7) (width 0.3) (layer "F.Cu") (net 7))
 (segment (start 136.265 95.915) (end 136.45 96.1) (width 0.3) (layer "F.Cu") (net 7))
 (segment (start 136.265 94.725) (end 136.265 95.915) (width 0.3) (layer "F.Cu") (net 7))
 (segment (start 145.5 97.7) (end 147.35 97.7) (width 0.3) (layer "F.Cu") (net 7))
 (segment (start 143.9 96.1) (end 145.5 97.7) (width 0.3) (layer "F.Cu") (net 7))
 (segment (start 137.895 98.64) (end 137.535 99) (width 0.3) (layer "F.Cu") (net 2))
 (segment (start 127.4625 97.75) (end 127.5125 97.7) (width 0.3) (layer "F.Cu") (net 2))
 (segment (start 137.535 99) (end 137.535 99.675) (width 0.3) (layer "F.Cu") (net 2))
 (segment (start 127.5125 97.7) (end 129.75 97.7) (width 0.3) (layer "F.Cu") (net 2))
 (segment (start 137.895 98.049219) (end 137.895 98.64) (width 0.3) (layer "F.Cu") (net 2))
 (segment (start 131.762501 97.65) (end 137.495781 97.65) (width 0.3) (layer "F.Cu") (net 2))
 (segment (start 131.187501 98.225) (end 131.762501 97.65) (width 0.3) (layer "F.Cu") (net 2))
 (segment (start 137.495781 97.65) (end 137.895 98.049219) (width 0.3) (layer "F.Cu") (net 2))
 (segment (start 130.4 98.225) (end 131.187501 98.225) (width 0.3) (layer "F.Cu") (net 2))
 (segment (start 130.275 98.225) (end 130.4 98.225) (width 0.3) (layer "F.Cu") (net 2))
 (segment (start 129.75 97.7) (end 130.275 98.225) (width 0.3) (layer "F.Cu") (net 2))
 (segment (start 127.5125 97.15) (end 129.775 97.15) (width 0.3) (layer "F.Cu") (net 14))
 (segment (start 138.445 97.821399) (end 138.445 98.64) (width 0.3) (layer "F.Cu") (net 14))
 (segment (start 130.4 96.525) (end 131.187501 96.525) (width 0.3) (layer "F.Cu") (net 14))
 (segment (start 138.445 98.64) (end 138.805 99) (width 0.3) (layer "F.Cu") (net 14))
 (segment (start 129.775 97.15) (end 130.4 96.525) (width 0.3) (layer "F.Cu") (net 14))
 (segment (start 131.762501 97.1) (end 137.723601 97.1) (width 0.3) (layer "F.Cu") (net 14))
 (segment (start 137.723601 97.1) (end 138.445 97.821399) (width 0.3) (layer "F.Cu") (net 14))
 (segment (start 131.187501 96.525) (end 131.762501 97.1) (width 0.3) (layer "F.Cu") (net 14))
 (segment (start 138.805 99) (end 138.805 99.675) (width 0.3) (layer "F.Cu") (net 14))
 (segment (start 127.4625 97.1) (end 127.5125 97.15) (width 0.3) (layer "F.Cu") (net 14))
 (segment (start 142.475 94.725) (end 142.5 94.7) (width 0.3) (layer "F.Cu") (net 13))
 (segment (start 141.345 94.725) (end 142.475 94.725) (width 0.3) (layer "F.Cu") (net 13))
 (via (at 142.5 94.7) (size 0.6) (drill 0.3) (layers "F.Cu" "B.Cu") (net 13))
 (segment (start 142.6 94.6) (end 150.1 94.6) (width 0.3) (layer "B.Cu") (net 13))
 (segment (start 151.85 96.35) (end 151.85 101.85) (width 0.3) (layer "B.Cu") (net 13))
 (segment (start 142.5 94.7) (end 142.6 94.6) (width 0.3) (layer "B.Cu") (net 13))
 (segment (start 149.95 103.75) (end 149.94 103.75) (width 0.3) (layer "B.Cu") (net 13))
 (segment (start 151.85 101.85) (end 149.95 103.75) (width 0.3) (layer "B.Cu") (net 13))
 (segment (start 150.1 94.6) (end 151.85 96.35) (width 0.3) (layer "B.Cu") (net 13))
 (segment (start 147.7125 99.2) (end 151.2875 99.2) (width 0.3) (layer "F.Cu") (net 3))
 (segment (start 151.2875 99.2) (end 151.6 99.5125) (width 0.3) (layer "F.Cu") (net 3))
 (segment (start 147.6375 95.775) (end 147.6625 95.8) (width 0.3) (layer "F.Cu") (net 6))
 (segment (start 147.6375 94.3) (end 147.6375 95.775) (width 0.3) (layer "F.Cu") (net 6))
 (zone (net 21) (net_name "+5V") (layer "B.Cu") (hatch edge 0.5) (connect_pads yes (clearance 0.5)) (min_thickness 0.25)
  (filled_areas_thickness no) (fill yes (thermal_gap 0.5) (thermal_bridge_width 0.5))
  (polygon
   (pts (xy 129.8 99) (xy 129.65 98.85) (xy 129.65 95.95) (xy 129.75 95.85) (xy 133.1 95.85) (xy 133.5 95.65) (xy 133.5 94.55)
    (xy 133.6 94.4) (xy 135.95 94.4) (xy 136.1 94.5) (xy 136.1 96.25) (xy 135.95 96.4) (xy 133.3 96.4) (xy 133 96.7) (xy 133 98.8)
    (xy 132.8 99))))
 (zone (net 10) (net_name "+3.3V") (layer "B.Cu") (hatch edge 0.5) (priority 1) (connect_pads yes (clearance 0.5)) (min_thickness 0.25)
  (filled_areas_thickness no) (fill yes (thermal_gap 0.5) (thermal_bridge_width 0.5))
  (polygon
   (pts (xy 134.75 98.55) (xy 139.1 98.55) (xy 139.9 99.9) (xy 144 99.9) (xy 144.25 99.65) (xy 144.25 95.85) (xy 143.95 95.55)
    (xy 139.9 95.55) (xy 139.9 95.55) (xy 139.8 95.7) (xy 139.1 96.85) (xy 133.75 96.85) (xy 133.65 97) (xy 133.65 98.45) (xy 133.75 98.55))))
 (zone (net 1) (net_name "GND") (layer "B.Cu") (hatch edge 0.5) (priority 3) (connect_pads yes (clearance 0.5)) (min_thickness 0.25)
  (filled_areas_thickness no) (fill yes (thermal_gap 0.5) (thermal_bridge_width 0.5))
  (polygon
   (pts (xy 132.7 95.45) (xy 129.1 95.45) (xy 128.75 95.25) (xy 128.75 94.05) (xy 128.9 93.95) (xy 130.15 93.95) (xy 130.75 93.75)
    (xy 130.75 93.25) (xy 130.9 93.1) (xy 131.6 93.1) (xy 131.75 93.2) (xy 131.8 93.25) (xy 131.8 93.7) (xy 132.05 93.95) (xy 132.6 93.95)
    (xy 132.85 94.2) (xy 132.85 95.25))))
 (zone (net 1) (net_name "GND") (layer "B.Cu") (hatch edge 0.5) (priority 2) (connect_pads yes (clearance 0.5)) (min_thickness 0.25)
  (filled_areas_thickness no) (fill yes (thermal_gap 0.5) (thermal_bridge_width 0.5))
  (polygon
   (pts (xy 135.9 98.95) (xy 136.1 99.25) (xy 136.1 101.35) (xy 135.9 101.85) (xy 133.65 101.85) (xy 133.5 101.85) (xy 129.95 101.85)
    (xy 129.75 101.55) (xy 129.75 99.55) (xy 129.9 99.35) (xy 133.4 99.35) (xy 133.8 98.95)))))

